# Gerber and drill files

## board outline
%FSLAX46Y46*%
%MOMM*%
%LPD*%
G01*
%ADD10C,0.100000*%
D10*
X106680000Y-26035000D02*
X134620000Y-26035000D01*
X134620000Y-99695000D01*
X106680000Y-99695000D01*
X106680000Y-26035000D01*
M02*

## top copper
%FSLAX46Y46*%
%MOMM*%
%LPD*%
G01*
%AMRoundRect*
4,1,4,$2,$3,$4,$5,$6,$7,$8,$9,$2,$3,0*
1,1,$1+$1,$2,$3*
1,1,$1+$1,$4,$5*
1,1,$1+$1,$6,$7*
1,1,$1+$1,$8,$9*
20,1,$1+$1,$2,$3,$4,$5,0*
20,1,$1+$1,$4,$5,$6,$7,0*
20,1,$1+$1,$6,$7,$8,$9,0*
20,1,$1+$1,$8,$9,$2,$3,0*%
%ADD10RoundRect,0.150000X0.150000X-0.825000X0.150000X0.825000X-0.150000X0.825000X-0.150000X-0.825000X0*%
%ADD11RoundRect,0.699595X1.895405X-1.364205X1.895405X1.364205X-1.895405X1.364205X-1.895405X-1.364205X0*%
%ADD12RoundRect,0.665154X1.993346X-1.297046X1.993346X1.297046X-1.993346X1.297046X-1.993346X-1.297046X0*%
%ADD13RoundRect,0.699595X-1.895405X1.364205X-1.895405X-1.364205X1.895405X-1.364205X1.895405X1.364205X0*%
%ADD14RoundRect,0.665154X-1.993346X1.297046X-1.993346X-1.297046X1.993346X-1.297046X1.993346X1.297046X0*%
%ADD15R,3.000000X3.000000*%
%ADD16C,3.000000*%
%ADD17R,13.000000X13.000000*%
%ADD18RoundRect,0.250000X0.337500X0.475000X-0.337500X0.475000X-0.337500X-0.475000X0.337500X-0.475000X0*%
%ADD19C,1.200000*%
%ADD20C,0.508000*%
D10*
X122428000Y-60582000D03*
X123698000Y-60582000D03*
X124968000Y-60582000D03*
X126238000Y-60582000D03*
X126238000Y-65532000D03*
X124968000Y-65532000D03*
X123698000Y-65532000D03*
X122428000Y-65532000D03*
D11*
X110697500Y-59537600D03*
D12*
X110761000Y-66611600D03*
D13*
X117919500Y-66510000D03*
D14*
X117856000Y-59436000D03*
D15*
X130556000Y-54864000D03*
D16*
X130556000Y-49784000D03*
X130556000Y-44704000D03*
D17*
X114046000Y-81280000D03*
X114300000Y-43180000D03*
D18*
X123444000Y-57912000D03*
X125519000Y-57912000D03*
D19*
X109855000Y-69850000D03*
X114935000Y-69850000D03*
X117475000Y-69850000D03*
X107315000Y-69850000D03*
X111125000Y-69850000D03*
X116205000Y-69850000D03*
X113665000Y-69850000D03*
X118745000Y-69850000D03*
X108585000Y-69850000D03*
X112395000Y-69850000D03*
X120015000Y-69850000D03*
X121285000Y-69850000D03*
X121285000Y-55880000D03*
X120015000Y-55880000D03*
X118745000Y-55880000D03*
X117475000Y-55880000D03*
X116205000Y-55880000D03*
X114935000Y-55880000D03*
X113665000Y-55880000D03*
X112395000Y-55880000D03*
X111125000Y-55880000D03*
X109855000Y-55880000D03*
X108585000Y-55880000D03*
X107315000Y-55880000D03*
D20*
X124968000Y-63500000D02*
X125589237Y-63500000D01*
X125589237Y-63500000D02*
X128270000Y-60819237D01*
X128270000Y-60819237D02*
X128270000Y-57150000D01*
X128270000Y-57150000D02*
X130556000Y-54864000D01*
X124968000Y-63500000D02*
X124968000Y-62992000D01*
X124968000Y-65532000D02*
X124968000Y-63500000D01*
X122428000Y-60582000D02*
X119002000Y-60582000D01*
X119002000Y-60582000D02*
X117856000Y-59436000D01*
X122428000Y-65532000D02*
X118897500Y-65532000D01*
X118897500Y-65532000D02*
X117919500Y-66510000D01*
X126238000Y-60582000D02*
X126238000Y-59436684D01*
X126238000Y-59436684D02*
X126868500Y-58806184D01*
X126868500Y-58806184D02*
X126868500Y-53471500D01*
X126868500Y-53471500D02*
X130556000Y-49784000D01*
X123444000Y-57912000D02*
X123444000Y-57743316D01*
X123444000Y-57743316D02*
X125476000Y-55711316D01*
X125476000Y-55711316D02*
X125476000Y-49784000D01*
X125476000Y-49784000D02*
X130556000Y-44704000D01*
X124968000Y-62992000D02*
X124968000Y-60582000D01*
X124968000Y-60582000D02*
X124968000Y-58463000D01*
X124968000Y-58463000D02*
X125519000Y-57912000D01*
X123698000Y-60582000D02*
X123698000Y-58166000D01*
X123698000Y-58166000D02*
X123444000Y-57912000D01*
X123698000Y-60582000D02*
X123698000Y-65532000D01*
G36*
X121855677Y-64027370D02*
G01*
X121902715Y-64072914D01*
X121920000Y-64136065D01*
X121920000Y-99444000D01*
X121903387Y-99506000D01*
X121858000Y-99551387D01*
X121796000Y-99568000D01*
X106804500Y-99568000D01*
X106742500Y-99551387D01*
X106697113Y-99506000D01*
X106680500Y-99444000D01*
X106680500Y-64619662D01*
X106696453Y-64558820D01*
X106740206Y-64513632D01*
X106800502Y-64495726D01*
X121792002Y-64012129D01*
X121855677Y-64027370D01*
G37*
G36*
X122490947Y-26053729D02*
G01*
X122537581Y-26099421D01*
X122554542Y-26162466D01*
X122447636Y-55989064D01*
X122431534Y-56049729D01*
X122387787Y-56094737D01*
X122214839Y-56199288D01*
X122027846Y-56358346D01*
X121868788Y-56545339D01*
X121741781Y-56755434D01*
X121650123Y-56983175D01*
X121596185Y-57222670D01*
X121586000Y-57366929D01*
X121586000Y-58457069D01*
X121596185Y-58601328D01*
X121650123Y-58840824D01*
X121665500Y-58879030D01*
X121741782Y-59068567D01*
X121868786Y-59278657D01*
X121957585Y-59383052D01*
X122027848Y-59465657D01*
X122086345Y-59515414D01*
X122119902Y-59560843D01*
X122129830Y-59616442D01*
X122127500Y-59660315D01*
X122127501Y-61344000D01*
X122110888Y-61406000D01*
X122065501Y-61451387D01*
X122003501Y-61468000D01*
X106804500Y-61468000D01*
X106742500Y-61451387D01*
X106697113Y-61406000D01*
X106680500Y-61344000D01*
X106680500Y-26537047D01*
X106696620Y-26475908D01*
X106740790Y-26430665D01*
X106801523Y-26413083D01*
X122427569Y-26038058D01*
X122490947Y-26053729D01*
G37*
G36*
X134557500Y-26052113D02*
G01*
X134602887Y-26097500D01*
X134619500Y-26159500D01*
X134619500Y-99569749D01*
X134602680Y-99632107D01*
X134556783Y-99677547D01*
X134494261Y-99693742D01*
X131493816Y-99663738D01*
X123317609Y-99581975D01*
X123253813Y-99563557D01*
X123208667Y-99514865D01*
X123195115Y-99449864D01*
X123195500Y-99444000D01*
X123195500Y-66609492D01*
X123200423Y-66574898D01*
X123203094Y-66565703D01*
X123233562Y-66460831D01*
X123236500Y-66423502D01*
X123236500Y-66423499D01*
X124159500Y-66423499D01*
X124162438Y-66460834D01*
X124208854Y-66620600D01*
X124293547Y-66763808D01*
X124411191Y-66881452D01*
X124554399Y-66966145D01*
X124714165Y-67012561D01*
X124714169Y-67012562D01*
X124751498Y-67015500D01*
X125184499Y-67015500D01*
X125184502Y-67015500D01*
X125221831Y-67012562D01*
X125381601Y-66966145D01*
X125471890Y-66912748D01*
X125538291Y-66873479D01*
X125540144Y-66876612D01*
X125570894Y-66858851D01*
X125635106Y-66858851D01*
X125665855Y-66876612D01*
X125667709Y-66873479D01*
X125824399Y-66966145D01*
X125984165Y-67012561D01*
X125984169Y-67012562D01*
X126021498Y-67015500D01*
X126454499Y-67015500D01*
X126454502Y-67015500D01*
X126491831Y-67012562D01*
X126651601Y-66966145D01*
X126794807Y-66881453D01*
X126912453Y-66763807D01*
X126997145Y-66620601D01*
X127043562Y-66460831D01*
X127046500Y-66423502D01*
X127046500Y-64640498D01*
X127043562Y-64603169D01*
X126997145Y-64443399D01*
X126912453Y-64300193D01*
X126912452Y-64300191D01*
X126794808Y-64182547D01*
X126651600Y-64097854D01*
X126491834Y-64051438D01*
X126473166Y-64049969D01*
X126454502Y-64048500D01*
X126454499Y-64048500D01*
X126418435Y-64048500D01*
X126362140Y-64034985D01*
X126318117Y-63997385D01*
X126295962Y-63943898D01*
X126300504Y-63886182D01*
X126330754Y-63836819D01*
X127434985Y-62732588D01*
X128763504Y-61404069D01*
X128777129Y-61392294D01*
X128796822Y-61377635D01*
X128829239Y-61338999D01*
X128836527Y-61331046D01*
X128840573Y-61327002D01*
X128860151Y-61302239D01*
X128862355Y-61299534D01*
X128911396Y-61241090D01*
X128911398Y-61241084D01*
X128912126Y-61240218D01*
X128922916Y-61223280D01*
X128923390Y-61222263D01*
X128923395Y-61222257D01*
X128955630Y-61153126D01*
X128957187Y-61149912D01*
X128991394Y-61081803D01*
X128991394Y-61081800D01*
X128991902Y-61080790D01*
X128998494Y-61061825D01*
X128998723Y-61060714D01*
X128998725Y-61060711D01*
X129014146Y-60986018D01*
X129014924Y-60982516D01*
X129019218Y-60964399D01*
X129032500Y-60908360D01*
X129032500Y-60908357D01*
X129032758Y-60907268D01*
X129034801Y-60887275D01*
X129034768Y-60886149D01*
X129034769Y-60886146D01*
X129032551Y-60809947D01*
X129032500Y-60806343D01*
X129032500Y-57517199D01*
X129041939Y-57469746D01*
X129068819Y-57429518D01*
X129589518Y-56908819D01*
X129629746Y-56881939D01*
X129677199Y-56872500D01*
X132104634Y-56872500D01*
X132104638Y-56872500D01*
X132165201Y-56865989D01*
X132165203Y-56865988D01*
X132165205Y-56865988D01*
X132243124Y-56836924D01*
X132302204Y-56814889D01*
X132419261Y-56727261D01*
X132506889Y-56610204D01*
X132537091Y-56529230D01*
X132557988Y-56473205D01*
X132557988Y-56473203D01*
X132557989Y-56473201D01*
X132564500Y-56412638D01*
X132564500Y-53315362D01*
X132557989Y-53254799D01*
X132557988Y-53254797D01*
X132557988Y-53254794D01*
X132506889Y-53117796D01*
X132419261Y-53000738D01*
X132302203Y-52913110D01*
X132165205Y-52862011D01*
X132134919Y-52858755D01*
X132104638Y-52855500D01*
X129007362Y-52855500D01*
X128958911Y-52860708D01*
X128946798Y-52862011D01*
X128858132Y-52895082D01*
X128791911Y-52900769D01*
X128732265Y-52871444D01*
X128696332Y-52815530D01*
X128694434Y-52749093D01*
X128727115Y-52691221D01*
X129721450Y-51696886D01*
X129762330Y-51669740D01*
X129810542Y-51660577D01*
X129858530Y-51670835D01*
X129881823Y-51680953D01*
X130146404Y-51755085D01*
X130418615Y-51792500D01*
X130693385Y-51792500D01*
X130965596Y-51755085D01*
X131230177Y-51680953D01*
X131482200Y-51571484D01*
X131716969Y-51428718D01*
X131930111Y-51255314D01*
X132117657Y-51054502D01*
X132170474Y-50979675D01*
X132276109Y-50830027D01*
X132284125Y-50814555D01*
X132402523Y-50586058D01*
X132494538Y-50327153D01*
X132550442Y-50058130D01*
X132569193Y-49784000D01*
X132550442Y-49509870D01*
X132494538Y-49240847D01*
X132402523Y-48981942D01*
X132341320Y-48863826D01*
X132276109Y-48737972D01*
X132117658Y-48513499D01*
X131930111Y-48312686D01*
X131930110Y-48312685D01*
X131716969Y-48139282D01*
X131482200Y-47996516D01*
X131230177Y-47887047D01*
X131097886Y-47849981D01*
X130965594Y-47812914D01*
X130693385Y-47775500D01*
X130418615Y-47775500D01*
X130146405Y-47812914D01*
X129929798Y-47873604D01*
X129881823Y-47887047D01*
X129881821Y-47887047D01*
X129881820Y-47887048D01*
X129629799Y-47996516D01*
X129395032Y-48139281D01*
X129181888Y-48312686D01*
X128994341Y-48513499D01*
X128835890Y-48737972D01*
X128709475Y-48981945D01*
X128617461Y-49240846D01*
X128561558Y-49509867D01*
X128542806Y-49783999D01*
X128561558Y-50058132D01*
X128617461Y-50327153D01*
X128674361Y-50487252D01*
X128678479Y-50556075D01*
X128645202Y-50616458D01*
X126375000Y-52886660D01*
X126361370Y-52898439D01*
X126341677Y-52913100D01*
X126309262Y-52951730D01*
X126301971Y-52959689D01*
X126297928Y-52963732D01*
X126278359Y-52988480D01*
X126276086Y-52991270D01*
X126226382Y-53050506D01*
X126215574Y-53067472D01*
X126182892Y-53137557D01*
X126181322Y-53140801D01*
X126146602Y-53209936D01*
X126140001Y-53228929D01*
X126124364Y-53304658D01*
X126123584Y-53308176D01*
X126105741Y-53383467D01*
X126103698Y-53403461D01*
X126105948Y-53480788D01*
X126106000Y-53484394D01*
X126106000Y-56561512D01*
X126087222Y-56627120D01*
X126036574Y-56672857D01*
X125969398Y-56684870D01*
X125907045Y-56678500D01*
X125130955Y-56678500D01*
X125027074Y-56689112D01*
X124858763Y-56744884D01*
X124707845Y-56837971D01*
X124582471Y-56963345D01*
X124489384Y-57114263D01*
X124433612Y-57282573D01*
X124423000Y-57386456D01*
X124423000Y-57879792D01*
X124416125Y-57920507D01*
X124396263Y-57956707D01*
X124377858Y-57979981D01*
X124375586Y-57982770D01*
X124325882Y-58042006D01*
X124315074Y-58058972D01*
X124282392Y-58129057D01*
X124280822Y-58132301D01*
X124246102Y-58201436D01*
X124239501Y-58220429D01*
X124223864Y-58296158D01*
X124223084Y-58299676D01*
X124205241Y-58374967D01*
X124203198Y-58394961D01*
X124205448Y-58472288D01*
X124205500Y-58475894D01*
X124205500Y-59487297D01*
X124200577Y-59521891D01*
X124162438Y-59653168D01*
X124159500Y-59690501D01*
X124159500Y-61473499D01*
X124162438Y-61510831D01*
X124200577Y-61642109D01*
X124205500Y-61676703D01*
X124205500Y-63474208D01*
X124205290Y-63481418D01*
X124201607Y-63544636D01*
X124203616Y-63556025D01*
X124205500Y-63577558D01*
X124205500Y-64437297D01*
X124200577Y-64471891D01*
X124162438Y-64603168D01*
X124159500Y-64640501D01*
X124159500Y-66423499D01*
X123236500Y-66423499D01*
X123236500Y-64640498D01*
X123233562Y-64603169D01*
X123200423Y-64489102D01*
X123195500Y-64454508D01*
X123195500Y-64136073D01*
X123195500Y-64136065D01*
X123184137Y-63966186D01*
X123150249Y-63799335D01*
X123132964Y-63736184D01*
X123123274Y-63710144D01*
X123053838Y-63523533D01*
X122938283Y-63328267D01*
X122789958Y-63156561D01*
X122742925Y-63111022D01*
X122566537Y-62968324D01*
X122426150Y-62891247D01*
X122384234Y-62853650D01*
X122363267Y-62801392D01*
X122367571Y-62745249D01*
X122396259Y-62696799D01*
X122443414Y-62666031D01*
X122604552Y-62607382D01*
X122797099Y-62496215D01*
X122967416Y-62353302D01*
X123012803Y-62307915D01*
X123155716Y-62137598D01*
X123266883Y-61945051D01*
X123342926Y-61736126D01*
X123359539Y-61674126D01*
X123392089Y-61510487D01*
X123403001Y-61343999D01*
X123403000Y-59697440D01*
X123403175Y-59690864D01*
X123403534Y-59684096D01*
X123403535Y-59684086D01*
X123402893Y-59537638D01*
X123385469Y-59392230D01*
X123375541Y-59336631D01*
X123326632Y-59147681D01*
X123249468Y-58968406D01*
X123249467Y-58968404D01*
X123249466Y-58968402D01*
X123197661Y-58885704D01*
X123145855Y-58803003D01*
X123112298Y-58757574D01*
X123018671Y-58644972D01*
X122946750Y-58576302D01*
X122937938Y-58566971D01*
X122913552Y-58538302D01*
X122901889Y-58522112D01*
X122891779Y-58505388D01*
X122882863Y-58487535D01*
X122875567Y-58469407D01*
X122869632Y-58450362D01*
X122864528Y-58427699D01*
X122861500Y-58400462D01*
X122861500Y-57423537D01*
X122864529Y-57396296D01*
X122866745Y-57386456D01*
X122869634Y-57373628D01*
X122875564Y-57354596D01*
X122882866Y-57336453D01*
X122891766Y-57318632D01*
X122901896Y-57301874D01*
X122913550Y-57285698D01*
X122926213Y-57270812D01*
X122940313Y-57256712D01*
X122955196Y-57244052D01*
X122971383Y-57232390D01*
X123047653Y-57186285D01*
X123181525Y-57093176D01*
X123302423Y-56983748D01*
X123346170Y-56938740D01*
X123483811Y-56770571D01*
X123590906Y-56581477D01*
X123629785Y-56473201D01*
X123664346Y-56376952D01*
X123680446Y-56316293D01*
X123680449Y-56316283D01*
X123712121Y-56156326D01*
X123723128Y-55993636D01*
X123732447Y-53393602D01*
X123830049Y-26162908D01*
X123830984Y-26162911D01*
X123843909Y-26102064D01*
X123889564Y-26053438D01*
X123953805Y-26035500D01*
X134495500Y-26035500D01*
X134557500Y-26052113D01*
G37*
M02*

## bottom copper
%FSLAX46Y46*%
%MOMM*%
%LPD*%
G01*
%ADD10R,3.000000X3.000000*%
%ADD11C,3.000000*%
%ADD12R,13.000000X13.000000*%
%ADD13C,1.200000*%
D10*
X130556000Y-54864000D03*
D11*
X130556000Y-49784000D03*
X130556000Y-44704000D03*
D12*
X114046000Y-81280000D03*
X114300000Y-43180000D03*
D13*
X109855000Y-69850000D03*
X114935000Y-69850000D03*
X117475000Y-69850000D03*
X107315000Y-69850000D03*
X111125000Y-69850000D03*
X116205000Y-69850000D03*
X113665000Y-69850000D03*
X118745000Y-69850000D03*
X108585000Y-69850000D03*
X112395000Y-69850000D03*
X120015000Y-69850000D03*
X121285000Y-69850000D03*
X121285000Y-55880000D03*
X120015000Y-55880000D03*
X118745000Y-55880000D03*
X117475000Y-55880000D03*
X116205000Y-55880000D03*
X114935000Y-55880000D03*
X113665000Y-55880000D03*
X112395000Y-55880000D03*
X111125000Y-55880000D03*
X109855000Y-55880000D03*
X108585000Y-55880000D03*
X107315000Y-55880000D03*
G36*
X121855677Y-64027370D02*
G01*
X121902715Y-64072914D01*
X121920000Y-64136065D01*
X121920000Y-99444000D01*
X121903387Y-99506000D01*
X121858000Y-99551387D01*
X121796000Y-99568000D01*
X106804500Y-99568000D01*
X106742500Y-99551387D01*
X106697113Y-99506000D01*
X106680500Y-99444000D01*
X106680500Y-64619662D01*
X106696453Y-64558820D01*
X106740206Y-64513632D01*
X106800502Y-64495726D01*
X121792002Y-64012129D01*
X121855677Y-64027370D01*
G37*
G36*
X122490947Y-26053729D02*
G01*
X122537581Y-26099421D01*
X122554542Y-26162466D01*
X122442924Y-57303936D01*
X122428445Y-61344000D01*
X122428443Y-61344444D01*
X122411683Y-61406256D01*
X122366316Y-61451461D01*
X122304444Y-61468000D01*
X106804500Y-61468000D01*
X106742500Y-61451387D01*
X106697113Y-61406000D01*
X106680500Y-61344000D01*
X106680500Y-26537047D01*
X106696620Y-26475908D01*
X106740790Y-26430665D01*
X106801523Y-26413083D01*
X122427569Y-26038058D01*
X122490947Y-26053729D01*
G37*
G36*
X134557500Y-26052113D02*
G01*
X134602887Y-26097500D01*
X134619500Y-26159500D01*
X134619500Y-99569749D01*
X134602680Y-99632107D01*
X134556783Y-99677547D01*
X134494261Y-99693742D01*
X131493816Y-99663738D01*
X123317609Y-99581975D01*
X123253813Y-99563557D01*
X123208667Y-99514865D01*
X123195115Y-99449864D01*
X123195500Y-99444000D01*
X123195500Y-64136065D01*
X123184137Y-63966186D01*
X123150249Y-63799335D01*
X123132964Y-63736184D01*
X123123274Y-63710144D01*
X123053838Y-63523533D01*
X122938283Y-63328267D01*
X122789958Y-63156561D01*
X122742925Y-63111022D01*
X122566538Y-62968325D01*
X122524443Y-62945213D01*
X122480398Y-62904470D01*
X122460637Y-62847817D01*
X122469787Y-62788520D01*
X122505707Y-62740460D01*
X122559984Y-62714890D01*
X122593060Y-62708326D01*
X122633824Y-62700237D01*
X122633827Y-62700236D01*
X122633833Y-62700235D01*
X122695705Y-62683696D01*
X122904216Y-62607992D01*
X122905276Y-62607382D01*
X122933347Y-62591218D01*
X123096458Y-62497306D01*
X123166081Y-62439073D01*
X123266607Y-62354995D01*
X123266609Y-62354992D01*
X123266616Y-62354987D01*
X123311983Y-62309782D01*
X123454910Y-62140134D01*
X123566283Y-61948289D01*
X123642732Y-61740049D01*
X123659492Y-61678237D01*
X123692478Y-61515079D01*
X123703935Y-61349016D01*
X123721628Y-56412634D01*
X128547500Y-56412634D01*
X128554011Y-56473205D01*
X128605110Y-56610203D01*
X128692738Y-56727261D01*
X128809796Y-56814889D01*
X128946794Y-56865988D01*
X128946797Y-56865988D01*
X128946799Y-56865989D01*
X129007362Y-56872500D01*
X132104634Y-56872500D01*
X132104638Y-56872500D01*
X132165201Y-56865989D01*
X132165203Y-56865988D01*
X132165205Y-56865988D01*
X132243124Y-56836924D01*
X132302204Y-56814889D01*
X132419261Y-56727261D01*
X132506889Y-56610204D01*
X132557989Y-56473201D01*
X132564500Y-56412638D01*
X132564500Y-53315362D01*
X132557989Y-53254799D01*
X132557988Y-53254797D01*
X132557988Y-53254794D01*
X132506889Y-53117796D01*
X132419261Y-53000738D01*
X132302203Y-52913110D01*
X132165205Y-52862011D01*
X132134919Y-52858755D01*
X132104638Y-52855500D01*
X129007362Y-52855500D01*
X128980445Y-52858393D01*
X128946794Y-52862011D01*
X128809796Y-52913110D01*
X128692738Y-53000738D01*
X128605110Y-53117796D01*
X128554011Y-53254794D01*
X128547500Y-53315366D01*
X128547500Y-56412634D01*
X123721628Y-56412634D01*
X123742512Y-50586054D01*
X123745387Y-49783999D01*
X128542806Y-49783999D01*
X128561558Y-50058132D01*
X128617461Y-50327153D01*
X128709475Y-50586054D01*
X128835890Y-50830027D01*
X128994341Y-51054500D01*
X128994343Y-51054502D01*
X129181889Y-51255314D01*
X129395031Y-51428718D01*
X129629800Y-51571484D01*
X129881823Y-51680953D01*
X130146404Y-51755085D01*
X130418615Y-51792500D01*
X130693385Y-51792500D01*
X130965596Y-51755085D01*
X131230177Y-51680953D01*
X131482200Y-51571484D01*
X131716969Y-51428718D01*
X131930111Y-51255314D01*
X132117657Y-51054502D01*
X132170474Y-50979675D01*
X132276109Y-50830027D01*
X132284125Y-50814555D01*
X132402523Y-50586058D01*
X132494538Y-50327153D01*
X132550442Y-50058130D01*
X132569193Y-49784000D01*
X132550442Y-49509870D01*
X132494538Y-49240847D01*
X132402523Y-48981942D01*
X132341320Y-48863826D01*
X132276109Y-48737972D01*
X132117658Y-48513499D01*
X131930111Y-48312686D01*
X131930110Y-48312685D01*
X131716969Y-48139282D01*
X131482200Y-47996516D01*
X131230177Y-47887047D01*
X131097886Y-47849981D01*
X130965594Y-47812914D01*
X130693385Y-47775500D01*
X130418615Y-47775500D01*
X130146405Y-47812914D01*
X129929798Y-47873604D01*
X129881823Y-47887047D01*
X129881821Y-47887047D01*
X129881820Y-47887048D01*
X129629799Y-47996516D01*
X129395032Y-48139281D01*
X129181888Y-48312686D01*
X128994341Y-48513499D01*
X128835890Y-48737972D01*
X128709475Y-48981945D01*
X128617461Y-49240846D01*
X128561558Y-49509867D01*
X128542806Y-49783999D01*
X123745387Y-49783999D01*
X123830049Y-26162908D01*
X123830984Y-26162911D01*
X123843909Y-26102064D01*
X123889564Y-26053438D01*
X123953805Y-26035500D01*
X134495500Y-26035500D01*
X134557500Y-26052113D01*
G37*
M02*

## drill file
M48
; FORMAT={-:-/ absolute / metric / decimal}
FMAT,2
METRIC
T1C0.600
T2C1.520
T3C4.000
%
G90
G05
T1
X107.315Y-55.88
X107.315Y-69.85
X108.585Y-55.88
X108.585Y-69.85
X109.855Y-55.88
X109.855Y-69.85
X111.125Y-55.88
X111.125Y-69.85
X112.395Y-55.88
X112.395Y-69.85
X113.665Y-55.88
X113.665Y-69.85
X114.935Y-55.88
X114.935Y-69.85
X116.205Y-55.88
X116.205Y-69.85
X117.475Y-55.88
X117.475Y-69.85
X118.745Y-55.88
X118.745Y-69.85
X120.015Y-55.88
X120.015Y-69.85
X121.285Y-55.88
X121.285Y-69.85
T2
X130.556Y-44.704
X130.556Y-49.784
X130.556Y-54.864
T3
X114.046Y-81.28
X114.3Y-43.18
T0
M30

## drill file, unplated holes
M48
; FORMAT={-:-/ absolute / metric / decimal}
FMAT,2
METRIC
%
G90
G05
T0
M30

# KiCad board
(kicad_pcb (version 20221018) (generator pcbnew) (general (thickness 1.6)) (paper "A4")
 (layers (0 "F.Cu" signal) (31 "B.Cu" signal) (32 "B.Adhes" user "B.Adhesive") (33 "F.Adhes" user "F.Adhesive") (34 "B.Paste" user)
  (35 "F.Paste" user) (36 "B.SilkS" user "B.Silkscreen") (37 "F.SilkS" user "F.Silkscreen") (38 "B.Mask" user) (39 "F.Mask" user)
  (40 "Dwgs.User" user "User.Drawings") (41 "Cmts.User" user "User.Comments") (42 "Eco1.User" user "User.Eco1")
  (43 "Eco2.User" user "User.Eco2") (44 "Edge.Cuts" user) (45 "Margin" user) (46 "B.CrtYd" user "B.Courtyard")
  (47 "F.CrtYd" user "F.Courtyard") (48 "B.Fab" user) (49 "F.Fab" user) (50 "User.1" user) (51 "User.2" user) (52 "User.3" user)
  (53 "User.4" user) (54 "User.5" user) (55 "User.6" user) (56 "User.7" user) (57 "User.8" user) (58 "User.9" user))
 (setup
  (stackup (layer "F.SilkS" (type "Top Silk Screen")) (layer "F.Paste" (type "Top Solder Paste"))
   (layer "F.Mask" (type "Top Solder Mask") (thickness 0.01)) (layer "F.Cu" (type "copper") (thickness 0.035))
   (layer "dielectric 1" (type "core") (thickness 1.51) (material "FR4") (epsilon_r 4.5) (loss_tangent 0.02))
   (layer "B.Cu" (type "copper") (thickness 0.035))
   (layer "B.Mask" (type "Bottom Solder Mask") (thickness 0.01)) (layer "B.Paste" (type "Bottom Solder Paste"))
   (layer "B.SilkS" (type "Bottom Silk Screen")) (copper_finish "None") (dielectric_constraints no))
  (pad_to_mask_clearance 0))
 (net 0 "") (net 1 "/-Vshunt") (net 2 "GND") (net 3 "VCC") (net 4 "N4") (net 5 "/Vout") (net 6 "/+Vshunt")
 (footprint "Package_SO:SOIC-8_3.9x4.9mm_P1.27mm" (layer "F.Cu") (at 124.333 63.057 90)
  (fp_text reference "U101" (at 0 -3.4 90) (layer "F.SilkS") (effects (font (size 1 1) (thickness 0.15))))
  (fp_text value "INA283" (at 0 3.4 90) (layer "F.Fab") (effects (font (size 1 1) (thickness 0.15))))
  (pad "1" smd roundrect (at -2.475 -1.905 90) (size 1.95 0.6) (layers "F.Cu" "F.Paste" "F.Mask") (roundrect_rratio 0.25) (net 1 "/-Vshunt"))
  (pad "2" smd roundrect (at -2.475 -0.635 90) (size 1.95 0.6) (layers "F.Cu" "F.Paste" "F.Mask") (roundrect_rratio 0.25) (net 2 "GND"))
  (pad "3" smd roundrect (at -2.475 0.635 90) (size 1.95 0.6) (layers "F.Cu" "F.Paste" "F.Mask") (roundrect_rratio 0.25) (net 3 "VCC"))
  (pad "4" smd roundrect (at -2.475 1.905 90) (size 1.95 0.6) (layers "F.Cu" "F.Paste" "F.Mask") (roundrect_rratio 0.25) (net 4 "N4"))
  (pad "5" smd roundrect (at 2.475 1.905 90) (size 1.95 0.6) (layers "F.Cu" "F.Paste" "F.Mask") (roundrect_rratio 0.25) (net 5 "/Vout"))
  (pad "6" smd roundrect (at 2.475 0.635 90) (size 1.95 0.6) (layers "F.Cu" "F.Paste" "F.Mask") (roundrect_rratio 0.25) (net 3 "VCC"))
  (pad "7" smd roundrect (at 2.475 -0.635 90) (size 1.95 0.6) (layers "F.Cu" "F.Paste" "F.Mask") (roundrect_rratio 0.25) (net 2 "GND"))
  (pad "8" smd roundrect (at 2.475 -1.905 90) (size 1.95 0.6) (layers "F.Cu" "F.Paste" "F.Mask") (roundrect_rratio 0.25) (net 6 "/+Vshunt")))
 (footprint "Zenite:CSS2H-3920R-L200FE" (layer "F.Cu") (at 110.7525 63.0238 90)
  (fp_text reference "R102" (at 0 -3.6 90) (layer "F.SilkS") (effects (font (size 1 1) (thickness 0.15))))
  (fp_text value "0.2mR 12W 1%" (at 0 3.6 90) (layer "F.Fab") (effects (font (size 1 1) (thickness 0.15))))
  (pad "1" smd roundrect (at -3.5878 0.0085 90) (size 3.9244 5.317) (layers "F.Cu" "F.Paste" "F.Mask") (roundrect_rratio 0.1694918969)
   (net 1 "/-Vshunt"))
  (pad "2" smd roundrect (at 3.4862 -0.055 90) (size 4.1276 5.19) (layers "F.Cu" "F.Paste" "F.Mask") (roundrect_rratio 0.1694919566)
   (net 6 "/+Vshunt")))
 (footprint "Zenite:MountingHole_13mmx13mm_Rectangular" (layer "F.Cu") (at 114.3 43.18)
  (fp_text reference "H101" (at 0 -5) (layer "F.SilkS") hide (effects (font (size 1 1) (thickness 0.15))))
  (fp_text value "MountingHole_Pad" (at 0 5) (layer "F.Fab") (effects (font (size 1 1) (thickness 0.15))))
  (pad "1" thru_hole rect (at 0 0) (size 13 13) (drill 4) (layers "*.Cu" "*.Mask") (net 6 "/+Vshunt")))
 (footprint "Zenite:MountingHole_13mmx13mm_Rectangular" (layer "F.Cu") (at 114.046 81.28)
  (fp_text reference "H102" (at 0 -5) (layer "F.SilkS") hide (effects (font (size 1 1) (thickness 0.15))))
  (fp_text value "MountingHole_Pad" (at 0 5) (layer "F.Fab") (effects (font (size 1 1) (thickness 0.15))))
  (pad "1" thru_hole rect (at 0 0) (size 13 13) (drill 4) (layers "*.Cu" "*.Mask") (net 1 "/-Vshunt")))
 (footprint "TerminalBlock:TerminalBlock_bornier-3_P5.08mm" (layer "F.Cu") (at 130.556 54.864 90)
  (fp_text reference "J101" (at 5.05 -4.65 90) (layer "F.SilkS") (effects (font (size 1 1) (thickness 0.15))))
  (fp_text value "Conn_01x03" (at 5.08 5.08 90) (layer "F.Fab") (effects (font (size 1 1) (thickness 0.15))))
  (pad "1" thru_hole rect (at 0 0 90) (size 3 3) (drill 1.52) (layers "*.Cu" "*.Mask") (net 3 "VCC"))
  (pad "2" thru_hole circle (at 5.08 0 90) (size 3 3) (drill 1.52) (layers "*.Cu" "*.Mask") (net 5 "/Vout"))
  (pad "3" thru_hole circle (at 10.16 0 90) (size 3 3) (drill 1.52) (layers "*.Cu" "*.Mask") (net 2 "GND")))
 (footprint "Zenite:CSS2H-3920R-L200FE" (layer "F.Cu") (at 117.8645 63.0238 -90)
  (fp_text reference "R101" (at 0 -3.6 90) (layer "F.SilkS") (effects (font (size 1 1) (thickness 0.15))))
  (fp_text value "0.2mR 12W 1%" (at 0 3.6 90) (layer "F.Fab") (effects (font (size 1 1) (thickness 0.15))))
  (pad "1" smd roundrect (at -3.5878 0.0085 270) (size 3.9244 5.317) (layers "F.Cu" "F.Paste" "F.Mask") (roundrect_rratio 0.1694918969)
   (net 6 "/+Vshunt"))
  (pad "2" smd roundrect (at 3.4862 -0.055 270) (size 4.1276 5.19) (layers "F.Cu" "F.Paste" "F.Mask") (roundrect_rratio 0.1694919566)
   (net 1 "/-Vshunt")))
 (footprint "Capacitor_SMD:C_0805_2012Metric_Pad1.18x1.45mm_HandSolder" (layer "F.Cu") (at 124.4815 57.912 180)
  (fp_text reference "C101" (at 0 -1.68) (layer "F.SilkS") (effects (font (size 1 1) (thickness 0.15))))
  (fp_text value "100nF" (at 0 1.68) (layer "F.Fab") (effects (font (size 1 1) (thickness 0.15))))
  (pad "1" smd roundrect (at -1.0375 0 180) (size 1.175 1.45) (layers "F.Cu" "F.Paste" "F.Mask") (roundrect_rratio 0.2127659574)
   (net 3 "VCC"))
  (pad "2" smd roundrect (at 1.0375 0 180) (size 1.175 1.45) (layers "F.Cu" "F.Paste" "F.Mask") (roundrect_rratio 0.2127659574)
   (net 2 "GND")))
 (gr_rect (start 106.68 26.035) (end 134.62 99.695) (stroke (width 0.1) (type default)) (fill none) (layer "Edge.Cuts"))
 (segment (start 124.968 60.582) (end 124.968 58.463) (width 0.508) (layer "F.Cu") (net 3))
 (segment (start 124.968 63.5) (end 125.589237 63.5) (width 0.508) (layer "F.Cu") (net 3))
 (segment (start 128.27 57.15) (end 130.556 54.864) (width 0.508) (layer "F.Cu") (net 3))
 (segment (start 128.27 60.819237) (end 128.27 57.15) (width 0.508) (layer "F.Cu") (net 3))
 (segment (start 124.968 62.992) (end 124.968 60.582) (width 0.508) (layer "F.Cu") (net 3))
 (segment (start 125.589237 63.5) (end 128.27 60.819237) (width 0.508) (layer "F.Cu") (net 3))
 (segment (start 124.968 65.532) (end 124.968 63.5) (width 0.508) (layer "F.Cu") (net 3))
 (segment (start 124.968 58.463) (end 125.519 57.912) (width 0.508) (layer "F.Cu") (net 3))
 (segment (start 124.968 63.5) (end 124.968 62.992) (width 0.508) (layer "F.Cu") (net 3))
 (segment (start 125.476 55.711316) (end 125.476 49.784) (width 0.508) (layer "F.Cu") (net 2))
 (segment (start 123.444 57.743316) (end 125.476 55.711316) (width 0.508) (layer "F.Cu") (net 2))
 (segment (start 125.476 49.784) (end 130.556 44.704) (width 0.508) (layer "F.Cu") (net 2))
 (segment (start 123.698 60.582) (end 123.698 65.532) (width 0.508) (layer "F.Cu") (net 2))
 (segment (start 123.698 60.582) (end 123.698 58.166) (width 0.508) (layer "F.Cu") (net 2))
 (segment (start 123.698 58.166) (end 123.444 57.912) (width 0.508) (layer "F.Cu") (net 2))
 (segment (start 123.444 57.912) (end 123.444 57.743316) (width 0.508) (layer "F.Cu") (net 2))
 (segment (start 119.002 60.582) (end 117.856 59.436) (width 0.508) (layer "F.Cu") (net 6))
 (segment (start 122.428 60.582) (end 119.002 60.582) (width 0.508) (layer "F.Cu") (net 6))
 (via (at 112.395 55.88) (size 1.2) (drill 0.6) (layers "F.Cu" "B.Cu") (free) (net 6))
 (via (at 113.665 55.88) (size 1.2) (drill 0.6) (layers "F.Cu" "B.Cu") (free) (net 6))
 (via (at 109.855 55.88) (size 1.2) (drill 0.6) (layers "F.Cu" "B.Cu") (free) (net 6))
 (via (at 118.745 55.88) (size 1.2) (drill 0.6) (layers "F.Cu" "B.Cu") (free) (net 6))
 (via (at 116.205 55.88) (size 1.2) (drill 0.6) (layers "F.Cu" "B.Cu") (free) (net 6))
 (via (at 107.315 55.88) (size 1.2) (drill 0.6) (layers "F.Cu" "B.Cu") (free) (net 6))
 (via (at 114.935 55.88) (size 1.2) (drill 0.6) (layers "F.Cu" "B.Cu") (free) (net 6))
 (via (at 108.585 55.88) (size 1.2) (drill 0.6) (layers "F.Cu" "B.Cu") (free) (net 6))
 (via (at 120.015 55.88) (size 1.2) (drill 0.6) (layers "F.Cu" "B.Cu") (free) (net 6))
 (via (at 121.285 55.88) (size 1.2) (drill 0.6) (layers "F.Cu" "B.Cu") (free) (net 6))
 (via (at 111.125 55.88) (size 1.2) (drill 0.6) (layers "F.Cu" "B.Cu") (free) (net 6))
 (via (at 117.475 55.88) (size 1.2) (drill 0.6) (layers "F.Cu" "B.Cu") (free) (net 6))
 (segment (start 118.8975 65.532) (end 117.9195 66.51) (width 0.508) (layer "F.Cu") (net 1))
 (segment (start 122.428 65.532) (end 118.8975 65.532) (width 0.508) (layer "F.Cu") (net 1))
 (via (at 120.015 69.85) (size 1.2) (drill 0.6) (layers "F.Cu" "B.Cu") (free) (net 1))
 (via (at 116.205 69.85) (size 1.2) (drill 0.6) (layers "F.Cu" "B.Cu") (free) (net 1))
 (via (at 107.315 69.85) (size 1.2) (drill 0.6) (layers "F.Cu" "B.Cu") (free) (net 1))
 (via (at 109.855 69.85) (size 1.2) (drill 0.6) (layers "F.Cu" "B.Cu") (free) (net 1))
 (via (at 117.475 69.85) (size 1.2) (drill 0.6) (layers "F.Cu" "B.Cu") (free) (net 1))
 (via (at 108.585 69.85) (size 1.2) (drill 0.6) (layers "F.Cu" "B.Cu") (free) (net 1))
 (via (at 114.935 69.85) (size 1.2) (drill 0.6) (layers "F.Cu" "B.Cu") (free) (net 1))
 (via (at 113.665 69.85) (size 1.2) (drill 0.6) (layers "F.Cu" "B.Cu") (free) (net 1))
 (via (at 121.285 69.85) (size 1.2) (drill 0.6) (layers "F.Cu" "B.Cu") (free) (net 1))
 (via (at 118.745 69.85) (size 1.2) (drill 0.6) (layers "F.Cu" "B.Cu") (free) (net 1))
 (via (at 112.395 69.85) (size 1.2) (drill 0.6) (layers "F.Cu" "B.Cu") (free) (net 1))
 (via (at 111.125 69.85) (size 1.2) (drill 0.6) (layers "F.Cu" "B.Cu") (free) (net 1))
 (segment (start 126.8685 58.806184) (end 126.8685 53.4715) (width 0.508) (layer "F.Cu") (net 5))
 (segment (start 126.238 59.436684) (end 126.8685 58.806184) (width 0.508) (layer "F.Cu") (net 5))
 (segment (start 126.8685 53.4715) (end 130.556 49.784) (width 0.508) (layer "F.Cu") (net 5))
 (segment (start 126.238 60.582) (end 126.238 59.436684) (width 0.508) (layer "F.Cu") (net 5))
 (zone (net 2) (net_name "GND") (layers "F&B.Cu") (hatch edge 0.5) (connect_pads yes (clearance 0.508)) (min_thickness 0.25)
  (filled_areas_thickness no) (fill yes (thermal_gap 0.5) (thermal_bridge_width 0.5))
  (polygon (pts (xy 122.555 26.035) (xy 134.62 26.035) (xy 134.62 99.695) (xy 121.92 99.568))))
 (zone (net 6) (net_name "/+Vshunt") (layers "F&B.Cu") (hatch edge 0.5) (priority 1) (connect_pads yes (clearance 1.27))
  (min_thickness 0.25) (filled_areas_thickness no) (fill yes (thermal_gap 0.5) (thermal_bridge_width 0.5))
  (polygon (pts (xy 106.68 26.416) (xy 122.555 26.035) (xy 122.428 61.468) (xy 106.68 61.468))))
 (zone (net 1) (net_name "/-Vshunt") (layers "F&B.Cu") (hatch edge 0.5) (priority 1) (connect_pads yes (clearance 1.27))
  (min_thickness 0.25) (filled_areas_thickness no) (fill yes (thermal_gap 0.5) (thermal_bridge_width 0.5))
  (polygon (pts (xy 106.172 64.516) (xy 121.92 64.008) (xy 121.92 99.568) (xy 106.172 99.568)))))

